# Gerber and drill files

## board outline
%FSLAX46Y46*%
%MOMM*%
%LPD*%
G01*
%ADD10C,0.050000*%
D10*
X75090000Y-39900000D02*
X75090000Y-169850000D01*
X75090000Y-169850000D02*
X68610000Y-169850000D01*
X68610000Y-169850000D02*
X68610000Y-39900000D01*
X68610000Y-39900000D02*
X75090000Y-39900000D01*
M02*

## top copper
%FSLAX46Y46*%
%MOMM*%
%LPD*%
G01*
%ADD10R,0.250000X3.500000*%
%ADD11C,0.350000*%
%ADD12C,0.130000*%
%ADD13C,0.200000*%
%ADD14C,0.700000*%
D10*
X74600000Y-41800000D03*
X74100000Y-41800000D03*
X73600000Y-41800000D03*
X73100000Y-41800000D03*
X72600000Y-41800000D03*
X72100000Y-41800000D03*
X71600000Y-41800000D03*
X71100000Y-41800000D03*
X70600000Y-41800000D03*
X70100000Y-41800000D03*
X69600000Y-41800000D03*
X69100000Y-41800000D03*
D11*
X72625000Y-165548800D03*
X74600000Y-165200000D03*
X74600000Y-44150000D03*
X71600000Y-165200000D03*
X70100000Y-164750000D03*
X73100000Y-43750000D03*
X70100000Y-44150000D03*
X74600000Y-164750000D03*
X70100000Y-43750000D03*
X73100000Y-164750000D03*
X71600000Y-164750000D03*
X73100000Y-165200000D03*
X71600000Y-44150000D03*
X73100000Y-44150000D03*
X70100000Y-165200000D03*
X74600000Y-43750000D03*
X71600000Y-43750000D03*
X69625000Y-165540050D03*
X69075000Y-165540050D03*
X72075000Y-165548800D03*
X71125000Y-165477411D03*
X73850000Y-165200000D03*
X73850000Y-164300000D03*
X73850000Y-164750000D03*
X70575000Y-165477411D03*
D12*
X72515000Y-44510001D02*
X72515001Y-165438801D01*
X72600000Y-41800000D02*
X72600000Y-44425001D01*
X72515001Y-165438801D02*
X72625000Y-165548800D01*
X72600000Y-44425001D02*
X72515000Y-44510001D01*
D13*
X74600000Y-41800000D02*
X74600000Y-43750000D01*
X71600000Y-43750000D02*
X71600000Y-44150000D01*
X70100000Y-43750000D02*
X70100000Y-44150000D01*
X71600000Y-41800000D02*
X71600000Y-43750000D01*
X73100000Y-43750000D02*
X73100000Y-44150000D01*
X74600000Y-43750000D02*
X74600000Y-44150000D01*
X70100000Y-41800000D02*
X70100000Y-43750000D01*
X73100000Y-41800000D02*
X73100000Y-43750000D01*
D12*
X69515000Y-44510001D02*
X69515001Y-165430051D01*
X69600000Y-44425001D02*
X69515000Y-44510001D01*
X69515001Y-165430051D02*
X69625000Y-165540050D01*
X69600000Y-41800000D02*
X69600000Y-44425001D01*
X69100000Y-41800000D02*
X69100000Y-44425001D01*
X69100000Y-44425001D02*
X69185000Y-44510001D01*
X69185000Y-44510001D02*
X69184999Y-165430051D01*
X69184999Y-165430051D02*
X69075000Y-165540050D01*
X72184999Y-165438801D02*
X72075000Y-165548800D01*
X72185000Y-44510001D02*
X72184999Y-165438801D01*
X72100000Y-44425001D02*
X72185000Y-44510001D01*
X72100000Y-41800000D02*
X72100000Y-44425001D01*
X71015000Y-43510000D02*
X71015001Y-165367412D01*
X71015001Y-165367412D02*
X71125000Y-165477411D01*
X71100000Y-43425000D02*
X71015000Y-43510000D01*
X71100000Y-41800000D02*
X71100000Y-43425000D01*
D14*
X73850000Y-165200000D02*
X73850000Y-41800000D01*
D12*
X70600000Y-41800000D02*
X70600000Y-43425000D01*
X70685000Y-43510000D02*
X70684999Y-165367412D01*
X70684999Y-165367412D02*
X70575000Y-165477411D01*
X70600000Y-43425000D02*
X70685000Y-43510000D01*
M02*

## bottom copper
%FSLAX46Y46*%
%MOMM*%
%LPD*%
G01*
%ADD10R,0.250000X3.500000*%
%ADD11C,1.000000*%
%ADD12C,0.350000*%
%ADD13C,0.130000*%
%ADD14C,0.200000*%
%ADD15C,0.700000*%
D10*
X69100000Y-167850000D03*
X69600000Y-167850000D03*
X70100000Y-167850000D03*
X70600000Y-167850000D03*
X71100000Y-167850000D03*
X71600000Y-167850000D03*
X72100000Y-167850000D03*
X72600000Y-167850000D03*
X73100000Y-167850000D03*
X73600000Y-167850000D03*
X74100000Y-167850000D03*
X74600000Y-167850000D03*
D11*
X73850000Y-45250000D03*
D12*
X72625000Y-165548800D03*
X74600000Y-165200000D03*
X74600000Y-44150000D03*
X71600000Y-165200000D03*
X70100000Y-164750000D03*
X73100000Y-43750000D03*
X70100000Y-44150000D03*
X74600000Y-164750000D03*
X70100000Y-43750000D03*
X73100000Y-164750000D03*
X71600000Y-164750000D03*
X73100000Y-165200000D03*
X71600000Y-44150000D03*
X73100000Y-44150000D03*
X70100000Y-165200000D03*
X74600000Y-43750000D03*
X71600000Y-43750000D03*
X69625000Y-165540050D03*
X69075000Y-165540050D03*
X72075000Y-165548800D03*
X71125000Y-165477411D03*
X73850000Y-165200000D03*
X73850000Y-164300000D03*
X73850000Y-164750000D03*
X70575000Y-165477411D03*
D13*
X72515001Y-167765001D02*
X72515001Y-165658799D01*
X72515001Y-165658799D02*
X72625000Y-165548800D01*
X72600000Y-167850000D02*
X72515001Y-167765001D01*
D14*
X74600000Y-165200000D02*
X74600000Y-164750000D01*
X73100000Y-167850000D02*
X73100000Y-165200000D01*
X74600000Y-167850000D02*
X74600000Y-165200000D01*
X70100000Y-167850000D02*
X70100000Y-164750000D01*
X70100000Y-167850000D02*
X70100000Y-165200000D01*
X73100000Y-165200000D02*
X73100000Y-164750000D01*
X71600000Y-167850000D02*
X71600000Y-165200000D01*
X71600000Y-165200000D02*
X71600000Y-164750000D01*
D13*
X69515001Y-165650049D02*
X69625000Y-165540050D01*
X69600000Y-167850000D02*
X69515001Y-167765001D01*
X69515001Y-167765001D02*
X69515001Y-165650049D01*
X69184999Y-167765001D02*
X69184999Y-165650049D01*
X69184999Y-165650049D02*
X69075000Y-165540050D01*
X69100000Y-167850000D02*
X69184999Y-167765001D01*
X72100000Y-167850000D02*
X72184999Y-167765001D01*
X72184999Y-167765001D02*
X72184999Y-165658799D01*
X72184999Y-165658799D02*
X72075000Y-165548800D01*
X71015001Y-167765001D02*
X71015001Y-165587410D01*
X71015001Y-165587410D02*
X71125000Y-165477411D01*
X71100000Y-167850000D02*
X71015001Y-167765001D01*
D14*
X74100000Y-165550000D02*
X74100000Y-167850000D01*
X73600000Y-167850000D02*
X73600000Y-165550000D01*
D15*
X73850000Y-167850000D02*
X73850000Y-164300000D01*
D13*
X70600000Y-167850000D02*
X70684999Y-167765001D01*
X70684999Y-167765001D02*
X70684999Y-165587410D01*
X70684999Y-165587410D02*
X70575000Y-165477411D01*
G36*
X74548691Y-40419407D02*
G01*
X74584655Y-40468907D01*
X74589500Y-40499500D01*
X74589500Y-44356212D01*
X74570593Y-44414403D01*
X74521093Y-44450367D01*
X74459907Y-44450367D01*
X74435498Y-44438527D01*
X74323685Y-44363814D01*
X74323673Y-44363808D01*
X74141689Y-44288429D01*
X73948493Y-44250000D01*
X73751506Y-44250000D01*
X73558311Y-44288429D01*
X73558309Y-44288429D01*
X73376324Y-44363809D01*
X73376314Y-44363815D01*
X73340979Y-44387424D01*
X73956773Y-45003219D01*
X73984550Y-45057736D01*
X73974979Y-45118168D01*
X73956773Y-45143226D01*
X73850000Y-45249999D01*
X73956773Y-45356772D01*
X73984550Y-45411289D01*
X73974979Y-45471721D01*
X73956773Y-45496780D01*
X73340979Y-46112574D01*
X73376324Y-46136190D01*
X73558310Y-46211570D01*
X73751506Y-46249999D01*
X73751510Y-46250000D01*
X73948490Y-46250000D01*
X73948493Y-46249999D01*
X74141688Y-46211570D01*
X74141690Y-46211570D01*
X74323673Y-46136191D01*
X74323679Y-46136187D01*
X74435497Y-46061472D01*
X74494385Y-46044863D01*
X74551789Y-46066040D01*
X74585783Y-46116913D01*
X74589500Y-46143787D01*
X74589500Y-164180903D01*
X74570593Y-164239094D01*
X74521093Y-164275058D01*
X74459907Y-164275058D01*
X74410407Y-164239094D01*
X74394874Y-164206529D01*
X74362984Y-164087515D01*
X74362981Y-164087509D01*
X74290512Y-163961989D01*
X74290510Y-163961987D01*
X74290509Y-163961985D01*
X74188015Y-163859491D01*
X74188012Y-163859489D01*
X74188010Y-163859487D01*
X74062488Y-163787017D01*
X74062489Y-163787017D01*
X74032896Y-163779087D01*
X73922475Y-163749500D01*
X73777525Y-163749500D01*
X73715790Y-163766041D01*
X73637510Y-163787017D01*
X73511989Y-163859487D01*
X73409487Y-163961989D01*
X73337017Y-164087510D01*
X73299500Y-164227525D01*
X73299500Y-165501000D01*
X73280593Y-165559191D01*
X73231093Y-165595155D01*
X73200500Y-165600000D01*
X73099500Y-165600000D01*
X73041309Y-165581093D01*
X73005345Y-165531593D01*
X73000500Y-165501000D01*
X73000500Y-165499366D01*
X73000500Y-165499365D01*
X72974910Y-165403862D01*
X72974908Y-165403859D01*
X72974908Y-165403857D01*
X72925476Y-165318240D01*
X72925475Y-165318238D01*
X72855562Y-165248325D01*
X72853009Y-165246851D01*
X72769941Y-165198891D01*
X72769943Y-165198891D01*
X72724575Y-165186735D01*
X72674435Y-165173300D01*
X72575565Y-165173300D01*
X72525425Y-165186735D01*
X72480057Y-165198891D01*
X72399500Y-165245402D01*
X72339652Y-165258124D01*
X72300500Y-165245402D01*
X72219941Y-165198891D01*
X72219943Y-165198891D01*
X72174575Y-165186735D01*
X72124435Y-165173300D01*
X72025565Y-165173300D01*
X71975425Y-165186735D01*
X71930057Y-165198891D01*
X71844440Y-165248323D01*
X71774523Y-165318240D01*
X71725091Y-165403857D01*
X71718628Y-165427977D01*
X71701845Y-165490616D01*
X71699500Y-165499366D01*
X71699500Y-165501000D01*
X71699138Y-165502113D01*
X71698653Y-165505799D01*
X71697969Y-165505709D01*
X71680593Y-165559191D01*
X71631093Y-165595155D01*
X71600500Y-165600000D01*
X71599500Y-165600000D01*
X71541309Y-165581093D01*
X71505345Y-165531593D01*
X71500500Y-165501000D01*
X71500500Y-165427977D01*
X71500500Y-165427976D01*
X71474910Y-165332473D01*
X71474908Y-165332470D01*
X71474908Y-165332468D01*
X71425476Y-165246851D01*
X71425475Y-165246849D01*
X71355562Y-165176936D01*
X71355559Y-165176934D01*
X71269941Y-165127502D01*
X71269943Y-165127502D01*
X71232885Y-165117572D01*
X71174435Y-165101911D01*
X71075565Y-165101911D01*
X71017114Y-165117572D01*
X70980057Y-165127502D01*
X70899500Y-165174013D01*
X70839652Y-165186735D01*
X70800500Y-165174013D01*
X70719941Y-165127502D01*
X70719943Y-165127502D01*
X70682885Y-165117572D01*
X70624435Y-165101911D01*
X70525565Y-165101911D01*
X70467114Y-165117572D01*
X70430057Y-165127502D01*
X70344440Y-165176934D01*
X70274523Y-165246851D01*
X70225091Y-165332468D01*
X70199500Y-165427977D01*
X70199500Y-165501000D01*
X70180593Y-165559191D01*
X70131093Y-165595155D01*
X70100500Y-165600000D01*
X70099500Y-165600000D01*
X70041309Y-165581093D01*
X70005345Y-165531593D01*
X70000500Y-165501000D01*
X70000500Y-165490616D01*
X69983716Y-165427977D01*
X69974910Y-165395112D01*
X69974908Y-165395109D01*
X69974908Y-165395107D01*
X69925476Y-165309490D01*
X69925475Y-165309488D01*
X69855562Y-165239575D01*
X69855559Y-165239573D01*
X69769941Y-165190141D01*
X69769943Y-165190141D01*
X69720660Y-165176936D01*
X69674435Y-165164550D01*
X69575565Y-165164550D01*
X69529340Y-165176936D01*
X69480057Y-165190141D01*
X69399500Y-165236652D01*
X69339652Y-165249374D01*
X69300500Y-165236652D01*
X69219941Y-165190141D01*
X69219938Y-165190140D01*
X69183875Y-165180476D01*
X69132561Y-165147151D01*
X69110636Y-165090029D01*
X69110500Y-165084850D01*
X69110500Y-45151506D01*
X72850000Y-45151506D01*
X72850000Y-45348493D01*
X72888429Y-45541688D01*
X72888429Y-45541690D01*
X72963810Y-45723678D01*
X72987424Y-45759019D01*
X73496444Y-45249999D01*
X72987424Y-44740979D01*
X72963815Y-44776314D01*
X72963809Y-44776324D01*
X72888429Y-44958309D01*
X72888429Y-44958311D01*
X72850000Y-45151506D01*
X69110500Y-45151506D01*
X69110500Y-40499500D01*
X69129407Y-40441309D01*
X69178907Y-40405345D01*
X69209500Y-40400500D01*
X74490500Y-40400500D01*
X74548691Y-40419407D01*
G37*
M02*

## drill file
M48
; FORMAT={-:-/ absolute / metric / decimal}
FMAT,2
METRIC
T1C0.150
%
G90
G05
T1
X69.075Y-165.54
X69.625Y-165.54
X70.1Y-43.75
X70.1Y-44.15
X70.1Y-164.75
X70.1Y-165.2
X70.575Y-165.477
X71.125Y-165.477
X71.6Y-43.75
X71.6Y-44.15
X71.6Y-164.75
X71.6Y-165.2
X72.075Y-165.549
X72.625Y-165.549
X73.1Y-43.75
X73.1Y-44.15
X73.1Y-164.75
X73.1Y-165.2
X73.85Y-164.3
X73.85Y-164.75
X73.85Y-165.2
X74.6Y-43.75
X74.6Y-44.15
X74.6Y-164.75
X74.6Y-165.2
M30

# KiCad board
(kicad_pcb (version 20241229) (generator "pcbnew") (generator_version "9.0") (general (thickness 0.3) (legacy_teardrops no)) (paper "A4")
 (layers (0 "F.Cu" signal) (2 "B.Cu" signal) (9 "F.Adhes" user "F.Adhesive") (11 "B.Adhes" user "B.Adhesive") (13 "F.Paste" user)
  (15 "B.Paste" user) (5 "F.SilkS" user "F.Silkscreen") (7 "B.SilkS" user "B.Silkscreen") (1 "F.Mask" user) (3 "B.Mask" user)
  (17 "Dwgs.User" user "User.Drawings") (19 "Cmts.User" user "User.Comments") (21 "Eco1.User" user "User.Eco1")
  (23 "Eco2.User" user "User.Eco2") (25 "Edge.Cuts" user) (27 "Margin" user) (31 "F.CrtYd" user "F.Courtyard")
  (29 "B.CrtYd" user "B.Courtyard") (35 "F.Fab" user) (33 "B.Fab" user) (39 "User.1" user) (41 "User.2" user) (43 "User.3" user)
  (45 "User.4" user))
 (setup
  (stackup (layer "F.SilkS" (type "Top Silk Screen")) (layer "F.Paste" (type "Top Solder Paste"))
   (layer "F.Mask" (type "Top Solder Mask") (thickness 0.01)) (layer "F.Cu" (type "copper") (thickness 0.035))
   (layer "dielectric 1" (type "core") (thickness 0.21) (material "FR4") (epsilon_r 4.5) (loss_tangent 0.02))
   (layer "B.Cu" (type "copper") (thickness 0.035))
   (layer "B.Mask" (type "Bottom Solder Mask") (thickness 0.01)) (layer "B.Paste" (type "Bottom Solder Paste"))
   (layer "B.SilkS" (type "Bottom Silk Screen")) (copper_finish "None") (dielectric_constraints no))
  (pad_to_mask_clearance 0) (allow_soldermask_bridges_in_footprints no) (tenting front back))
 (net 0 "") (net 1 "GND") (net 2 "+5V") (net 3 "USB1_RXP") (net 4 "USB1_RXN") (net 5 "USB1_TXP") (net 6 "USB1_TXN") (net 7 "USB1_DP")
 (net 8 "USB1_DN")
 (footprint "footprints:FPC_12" (layer "F.Cu") (at 71.85 41.8)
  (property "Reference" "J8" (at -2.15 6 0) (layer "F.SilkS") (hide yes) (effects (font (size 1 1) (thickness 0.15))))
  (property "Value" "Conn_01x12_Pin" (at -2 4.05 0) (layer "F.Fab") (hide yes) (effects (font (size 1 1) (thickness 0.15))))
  (pad "1" smd rect (at 2.75 0) (size 0.25 3.5) (layers "F.Cu" "F.Mask" "F.Paste") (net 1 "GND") (thermal_bridge_angle 45))
  (pad "2" smd rect (at 2.25 0) (size 0.25 3.5) (layers "F.Cu" "F.Mask" "F.Paste") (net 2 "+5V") (thermal_bridge_angle 45))
  (pad "3" smd rect (at 1.75 0) (size 0.25 3.5) (layers "F.Cu" "F.Mask" "F.Paste") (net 2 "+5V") (thermal_bridge_angle 45))
  (pad "4" smd rect (at 1.25 0) (size 0.25 3.5) (layers "F.Cu" "F.Mask" "F.Paste") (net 1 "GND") (thermal_bridge_angle 45))
  (pad "5" smd rect (at 0.75 0) (size 0.25 3.5) (layers "F.Cu" "F.Mask" "F.Paste") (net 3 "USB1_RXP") (thermal_bridge_angle 45))
  (pad "6" smd rect (at 0.25 0) (size 0.25 3.5) (layers "F.Cu" "F.Mask" "F.Paste") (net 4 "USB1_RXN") (thermal_bridge_angle 45))
  (pad "7" smd rect (at -0.25 0) (size 0.25 3.5) (layers "F.Cu" "F.Mask" "F.Paste") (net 1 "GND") (thermal_bridge_angle 45))
  (pad "8" smd rect (at -0.75 0) (size 0.25 3.5) (layers "F.Cu" "F.Mask" "F.Paste") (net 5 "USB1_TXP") (thermal_bridge_angle 45))
  (pad "9" smd rect (at -1.25 0) (size 0.25 3.5) (layers "F.Cu" "F.Mask" "F.Paste") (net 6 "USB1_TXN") (thermal_bridge_angle 45))
  (pad "10" smd rect (at -1.75 0) (size 0.25 3.5) (layers "F.Cu" "F.Mask" "F.Paste") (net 1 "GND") (thermal_bridge_angle 45))
  (pad "11" smd rect (at -2.25 0) (size 0.25 3.5) (layers "F.Cu" "F.Mask" "F.Paste") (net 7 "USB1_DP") (thermal_bridge_angle 45))
  (pad "12" smd rect (at -2.75 0) (size 0.25 3.5) (layers "F.Cu" "F.Mask" "F.Paste") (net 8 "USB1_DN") (thermal_bridge_angle 45)))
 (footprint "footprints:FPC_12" (layer "B.Cu") (at 71.85 167.85 180)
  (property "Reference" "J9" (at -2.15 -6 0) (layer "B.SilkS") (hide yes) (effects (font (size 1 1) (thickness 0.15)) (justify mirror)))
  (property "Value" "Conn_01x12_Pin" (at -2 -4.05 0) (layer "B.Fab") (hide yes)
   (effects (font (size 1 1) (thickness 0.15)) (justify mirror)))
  (pad "1" smd rect (at 2.75 0 180) (size 0.25 3.5) (layers "B.Cu" "B.Mask" "B.Paste") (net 8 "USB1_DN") (thermal_bridge_angle 45))
  (pad "2" smd rect (at 2.25 0 180) (size 0.25 3.5) (layers "B.Cu" "B.Mask" "B.Paste") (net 7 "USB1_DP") (thermal_bridge_angle 45))
  (pad "3" smd rect (at 1.75 0 180) (size 0.25 3.5) (layers "B.Cu" "B.Mask" "B.Paste") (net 1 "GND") (thermal_bridge_angle 45))
  (pad "4" smd rect (at 1.25 0 180) (size 0.25 3.5) (layers "B.Cu" "B.Mask" "B.Paste") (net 6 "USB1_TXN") (thermal_bridge_angle 45))
  (pad "5" smd rect (at 0.75 0 180) (size 0.25 3.5) (layers "B.Cu" "B.Mask" "B.Paste") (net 5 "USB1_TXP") (thermal_bridge_angle 45))
  (pad "6" smd rect (at 0.25 0 180) (size 0.25 3.5) (layers "B.Cu" "B.Mask" "B.Paste") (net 1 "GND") (thermal_bridge_angle 45))
  (pad "7" smd rect (at -0.25 0 180) (size 0.25 3.5) (layers "B.Cu" "B.Mask" "B.Paste") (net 4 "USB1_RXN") (thermal_bridge_angle 45))
  (pad "8" smd rect (at -0.75 0 180) (size 0.25 3.5) (layers "B.Cu" "B.Mask" "B.Paste") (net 3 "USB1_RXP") (thermal_bridge_angle 45))
  (pad "9" smd rect (at -1.25 0 180) (size 0.25 3.5) (layers "B.Cu" "B.Mask" "B.Paste") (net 1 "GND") (thermal_bridge_angle 45))
  (pad "10" smd rect (at -1.75 0 180) (size 0.25 3.5) (layers "B.Cu" "B.Mask" "B.Paste") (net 2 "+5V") (thermal_bridge_angle 45))
  (pad "11" smd rect (at -2.25 0 180) (size 0.25 3.5) (layers "B.Cu" "B.Mask" "B.Paste") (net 2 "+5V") (thermal_bridge_angle 45))
  (pad "12" smd rect (at -2.75 0 180) (size 0.25 3.5) (layers "B.Cu" "B.Mask" "B.Paste") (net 1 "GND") (thermal_bridge_angle 45)))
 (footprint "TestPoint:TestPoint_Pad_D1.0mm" (layer "B.Cu") (at 73.85 45.25 180)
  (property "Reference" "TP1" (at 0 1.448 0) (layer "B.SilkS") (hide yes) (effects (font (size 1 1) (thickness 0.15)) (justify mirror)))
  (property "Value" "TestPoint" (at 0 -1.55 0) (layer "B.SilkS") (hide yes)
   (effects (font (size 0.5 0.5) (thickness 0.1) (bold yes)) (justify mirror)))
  (pad "1" smd circle (at 0 0 180) (size 1 1) (layers "B.Cu" "B.Mask") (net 1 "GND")))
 (gr_line (start 75.09 39.9) (end 75.09 169.85) (stroke (width 0.05) (type solid)) (layer "Edge.Cuts"))
 (gr_line (start 75.09 169.85) (end 68.61 169.85) (stroke (width 0.05) (type solid)) (layer "Edge.Cuts"))
 (gr_line (start 68.61 169.85) (end 68.61 39.9) (stroke (width 0.05) (type solid)) (layer "Edge.Cuts"))
 (gr_line (start 68.61 39.9) (end 75.09 39.9) (stroke (width 0.05) (type solid)) (layer "Edge.Cuts"))
 (segment (start 72.515 44.510001) (end 72.515001 165.438801) (width 0.13) (layer "F.Cu") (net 3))
 (segment (start 72.6 41.8) (end 72.6 44.425001) (width 0.13) (layer "F.Cu") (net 3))
 (segment (start 72.515001 165.438801) (end 72.625 165.5488) (width 0.13) (layer "F.Cu") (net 3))
 (segment (start 72.6 44.425001) (end 72.515 44.510001) (width 0.13) (layer "F.Cu") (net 3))
 (via (at 72.625 165.5488) (size 0.35) (drill 0.15) (layers "F.Cu" "B.Cu") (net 3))
 (segment (start 72.515001 167.765001) (end 72.515001 165.658799) (width 0.13) (layer "B.Cu") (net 3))
 (segment (start 72.515001 165.658799) (end 72.625 165.5488) (width 0.13) (layer "B.Cu") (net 3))
 (segment (start 72.6 167.85) (end 72.515001 167.765001) (width 0.13) (layer "B.Cu") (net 3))
 (segment (start 74.6 41.8) (end 74.6 43.75) (width 0.2) (layer "F.Cu") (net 1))
 (segment (start 71.6 43.75) (end 71.6 44.15) (width 0.2) (layer "F.Cu") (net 1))
 (segment (start 70.1 43.75) (end 70.1 44.15) (width 0.2) (layer "F.Cu") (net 1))
 (segment (start 71.6 41.8) (end 71.6 43.75) (width 0.2) (layer "F.Cu") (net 1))
 (segment (start 73.1 43.75) (end 73.1 44.15) (width 0.2) (layer "F.Cu") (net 1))
 (segment (start 74.6 43.75) (end 74.6 44.15) (width 0.2) (layer "F.Cu") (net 1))
 (segment (start 70.1 41.8) (end 70.1 43.75) (width 0.2) (layer "F.Cu") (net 1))
 (segment (start 73.1 41.8) (end 73.1 43.75) (width 0.2) (layer "F.Cu") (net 1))
 (via (at 74.6 165.2) (size 0.35) (drill 0.15) (layers "F.Cu" "B.Cu") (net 1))
 (via (at 74.6 44.15) (size 0.35) (drill 0.15) (layers "F.Cu" "B.Cu") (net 1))
 (via (at 71.6 165.2) (size 0.35) (drill 0.15) (layers "F.Cu" "B.Cu") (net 1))
 (via (at 70.1 164.75) (size 0.35) (drill 0.15) (layers "F.Cu" "B.Cu") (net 1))
 (via (at 73.1 43.75) (size 0.35) (drill 0.15) (layers "F.Cu" "B.Cu") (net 1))
 (via (at 70.1 44.15) (size 0.35) (drill 0.15) (layers "F.Cu" "B.Cu") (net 1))
 (via (at 74.6 164.75) (size 0.35) (drill 0.15) (layers "F.Cu" "B.Cu") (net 1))
 (via (at 70.1 43.75) (size 0.35) (drill 0.15) (layers "F.Cu" "B.Cu") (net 1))
 (via (at 73.1 164.75) (size 0.35) (drill 0.15) (layers "F.Cu" "B.Cu") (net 1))
 (via (at 71.6 164.75) (size 0.35) (drill 0.15) (layers "F.Cu" "B.Cu") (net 1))
 (via (at 73.1 165.2) (size 0.35) (drill 0.15) (layers "F.Cu" "B.Cu") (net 1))
 (via (at 71.6 44.15) (size 0.35) (drill 0.15) (layers "F.Cu" "B.Cu") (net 1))
 (via (at 73.1 44.15) (size 0.35) (drill 0.15) (layers "F.Cu" "B.Cu") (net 1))
 (via (at 70.1 165.2) (size 0.35) (drill 0.15) (layers "F.Cu" "B.Cu") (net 1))
 (via (at 74.6 43.75) (size 0.35) (drill 0.15) (layers "F.Cu" "B.Cu") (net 1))
 (via (at 71.6 43.75) (size 0.35) (drill 0.15) (layers "F.Cu" "B.Cu") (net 1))
 (segment (start 74.6 165.2) (end 74.6 164.75) (width 0.2) (layer "B.Cu") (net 1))
 (segment (start 73.1 167.85) (end 73.1 165.2) (width 0.2) (layer "B.Cu") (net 1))
 (segment (start 74.6 167.85) (end 74.6 165.2) (width 0.2) (layer "B.Cu") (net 1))
 (segment (start 70.1 167.85) (end 70.1 164.75) (width 0.2) (layer "B.Cu") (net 1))
 (segment (start 70.1 167.85) (end 70.1 165.2) (width 0.2) (layer "B.Cu") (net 1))
 (segment (start 73.1 165.2) (end 73.1 164.75) (width 0.2) (layer "B.Cu") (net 1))
 (segment (start 71.6 167.85) (end 71.6 165.2) (width 0.2) (layer "B.Cu") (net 1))
 (segment (start 71.6 165.2) (end 71.6 164.75) (width 0.2) (layer "B.Cu") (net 1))
 (segment (start 69.515 44.510001) (end 69.515001 165.430051) (width 0.13) (layer "F.Cu") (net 7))
 (segment (start 69.6 44.425001) (end 69.515 44.510001) (width 0.13) (layer "F.Cu") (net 7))
 (segment (start 69.515001 165.430051) (end 69.625 165.54005) (width 0.13) (layer "F.Cu") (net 7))
 (segment (start 69.6 41.8) (end 69.6 44.425001) (width 0.13) (layer "F.Cu") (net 7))
 (via (at 69.625 165.54005) (size 0.35) (drill 0.15) (layers "F.Cu" "B.Cu") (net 7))
 (segment (start 69.515001 165.650049) (end 69.625 165.54005) (width 0.13) (layer "B.Cu") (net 7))
 (segment (start 69.6 167.85) (end 69.515001 167.765001) (width 0.13) (layer "B.Cu") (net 7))
 (segment (start 69.515001 167.765001) (end 69.515001 165.650049) (width 0.13) (layer "B.Cu") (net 7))
 (segment (start 69.1 41.8) (end 69.1 44.425001) (width 0.13) (layer "F.Cu") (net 8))
 (segment (start 69.1 44.425001) (end 69.185 44.510001) (width 0.13) (layer "F.Cu") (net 8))
 (segment (start 69.185 44.510001) (end 69.184999 165.430051) (width 0.13) (layer "F.Cu") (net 8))
 (segment (start 69.184999 165.430051) (end 69.075 165.54005) (width 0.13) (layer "F.Cu") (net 8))
 (via (at 69.075 165.54005) (size 0.35) (drill 0.15) (layers "F.Cu" "B.Cu") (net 8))
 (segment (start 69.184999 167.765001) (end 69.184999 165.650049) (width 0.13) (layer "B.Cu") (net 8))
 (segment (start 69.184999 165.650049) (end 69.075 165.54005) (width 0.13) (layer "B.Cu") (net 8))
 (segment (start 69.1 167.85) (end 69.184999 167.765001) (width 0.13) (layer "B.Cu") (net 8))
 (segment (start 72.184999 165.438801) (end 72.075 165.5488) (width 0.13) (layer "F.Cu") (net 4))
 (segment (start 72.185 44.510001) (end 72.184999 165.438801) (width 0.13) (layer "F.Cu") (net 4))
 (segment (start 72.1 44.425001) (end 72.185 44.510001) (width 0.13) (layer "F.Cu") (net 4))
 (segment (start 72.1 41.8) (end 72.1 44.425001) (width 0.13) (layer "F.Cu") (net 4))
 (via (at 72.075 165.5488) (size 0.35) (drill 0.15) (layers "F.Cu" "B.Cu") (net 4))
 (segment (start 72.1 167.85) (end 72.184999 167.765001) (width 0.13) (layer "B.Cu") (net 4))
 (segment (start 72.184999 167.765001) (end 72.184999 165.658799) (width 0.13) (layer "B.Cu") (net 4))
 (segment (start 72.184999 165.658799) (end 72.075 165.5488) (width 0.13) (layer "B.Cu") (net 4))
 (segment (start 71.015 43.51) (end 71.015001 165.367412) (width 0.13) (layer "F.Cu") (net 5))
 (segment (start 71.015001 165.367412) (end 71.125 165.477411) (width 0.13) (layer "F.Cu") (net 5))
 (segment (start 71.1 43.425) (end 71.015 43.51) (width 0.13) (layer "F.Cu") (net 5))
 (segment (start 71.1 41.8) (end 71.1 43.425) (width 0.13) (layer "F.Cu") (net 5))
 (via (at 71.125 165.477411) (size 0.35) (drill 0.15) (layers "F.Cu" "B.Cu") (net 5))
 (segment (start 71.015001 167.765001) (end 71.015001 165.58741) (width 0.13) (layer "B.Cu") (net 5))
 (segment (start 71.015001 165.58741) (end 71.125 165.477411) (width 0.13) (layer "B.Cu") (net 5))
 (segment (start 71.1 167.85) (end 71.015001 167.765001) (width 0.13) (layer "B.Cu") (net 5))
 (segment (start 73.85 165.2) (end 73.85 41.8) (width 0.7) (layer "F.Cu") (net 2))
 (via (at 73.85 165.2) (size 0.35) (drill 0.15) (layers "F.Cu" "B.Cu") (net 2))
 (via (at 73.85 164.3) (size 0.35) (drill 0.15) (layers "F.Cu" "B.Cu") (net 2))
 (via (at 73.85 164.75) (size 0.35) (drill 0.15) (layers "F.Cu" "B.Cu") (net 2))
 (segment (start 74.1 165.55) (end 74.1 167.85) (width 0.2) (layer "B.Cu") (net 2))
 (segment (start 73.6 167.85) (end 73.6 165.55) (width 0.2) (layer "B.Cu") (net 2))
 (segment (start 73.85 167.85) (end 73.85 164.3) (width 0.7) (layer "B.Cu") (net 2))
 (segment (start 70.6 41.8) (end 70.6 43.425) (width 0.13) (layer "F.Cu") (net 6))
 (segment (start 70.685 43.51) (end 70.684999 165.367412) (width 0.13) (layer "F.Cu") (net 6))
 (segment (start 70.684999 165.367412) (end 70.575 165.477411) (width 0.13) (layer "F.Cu") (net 6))
 (segment (start 70.6 43.425) (end 70.685 43.51) (width 0.13) (layer "F.Cu") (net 6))
 (via (at 70.575 165.477411) (size 0.35) (drill 0.15) (layers "F.Cu" "B.Cu") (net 6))
 (segment (start 70.6 167.85) (end 70.684999 167.765001) (width 0.13) (layer "B.Cu") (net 6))
 (segment (start 70.684999 167.765001) (end 70.684999 165.58741) (width 0.13) (layer "B.Cu") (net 6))
 (segment (start 70.684999 165.58741) (end 70.575 165.477411) (width 0.13) (layer "B.Cu") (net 6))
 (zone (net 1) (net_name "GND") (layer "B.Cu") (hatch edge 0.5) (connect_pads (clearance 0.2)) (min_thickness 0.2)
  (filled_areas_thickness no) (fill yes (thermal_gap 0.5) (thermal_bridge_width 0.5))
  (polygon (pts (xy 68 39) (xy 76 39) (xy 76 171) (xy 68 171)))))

